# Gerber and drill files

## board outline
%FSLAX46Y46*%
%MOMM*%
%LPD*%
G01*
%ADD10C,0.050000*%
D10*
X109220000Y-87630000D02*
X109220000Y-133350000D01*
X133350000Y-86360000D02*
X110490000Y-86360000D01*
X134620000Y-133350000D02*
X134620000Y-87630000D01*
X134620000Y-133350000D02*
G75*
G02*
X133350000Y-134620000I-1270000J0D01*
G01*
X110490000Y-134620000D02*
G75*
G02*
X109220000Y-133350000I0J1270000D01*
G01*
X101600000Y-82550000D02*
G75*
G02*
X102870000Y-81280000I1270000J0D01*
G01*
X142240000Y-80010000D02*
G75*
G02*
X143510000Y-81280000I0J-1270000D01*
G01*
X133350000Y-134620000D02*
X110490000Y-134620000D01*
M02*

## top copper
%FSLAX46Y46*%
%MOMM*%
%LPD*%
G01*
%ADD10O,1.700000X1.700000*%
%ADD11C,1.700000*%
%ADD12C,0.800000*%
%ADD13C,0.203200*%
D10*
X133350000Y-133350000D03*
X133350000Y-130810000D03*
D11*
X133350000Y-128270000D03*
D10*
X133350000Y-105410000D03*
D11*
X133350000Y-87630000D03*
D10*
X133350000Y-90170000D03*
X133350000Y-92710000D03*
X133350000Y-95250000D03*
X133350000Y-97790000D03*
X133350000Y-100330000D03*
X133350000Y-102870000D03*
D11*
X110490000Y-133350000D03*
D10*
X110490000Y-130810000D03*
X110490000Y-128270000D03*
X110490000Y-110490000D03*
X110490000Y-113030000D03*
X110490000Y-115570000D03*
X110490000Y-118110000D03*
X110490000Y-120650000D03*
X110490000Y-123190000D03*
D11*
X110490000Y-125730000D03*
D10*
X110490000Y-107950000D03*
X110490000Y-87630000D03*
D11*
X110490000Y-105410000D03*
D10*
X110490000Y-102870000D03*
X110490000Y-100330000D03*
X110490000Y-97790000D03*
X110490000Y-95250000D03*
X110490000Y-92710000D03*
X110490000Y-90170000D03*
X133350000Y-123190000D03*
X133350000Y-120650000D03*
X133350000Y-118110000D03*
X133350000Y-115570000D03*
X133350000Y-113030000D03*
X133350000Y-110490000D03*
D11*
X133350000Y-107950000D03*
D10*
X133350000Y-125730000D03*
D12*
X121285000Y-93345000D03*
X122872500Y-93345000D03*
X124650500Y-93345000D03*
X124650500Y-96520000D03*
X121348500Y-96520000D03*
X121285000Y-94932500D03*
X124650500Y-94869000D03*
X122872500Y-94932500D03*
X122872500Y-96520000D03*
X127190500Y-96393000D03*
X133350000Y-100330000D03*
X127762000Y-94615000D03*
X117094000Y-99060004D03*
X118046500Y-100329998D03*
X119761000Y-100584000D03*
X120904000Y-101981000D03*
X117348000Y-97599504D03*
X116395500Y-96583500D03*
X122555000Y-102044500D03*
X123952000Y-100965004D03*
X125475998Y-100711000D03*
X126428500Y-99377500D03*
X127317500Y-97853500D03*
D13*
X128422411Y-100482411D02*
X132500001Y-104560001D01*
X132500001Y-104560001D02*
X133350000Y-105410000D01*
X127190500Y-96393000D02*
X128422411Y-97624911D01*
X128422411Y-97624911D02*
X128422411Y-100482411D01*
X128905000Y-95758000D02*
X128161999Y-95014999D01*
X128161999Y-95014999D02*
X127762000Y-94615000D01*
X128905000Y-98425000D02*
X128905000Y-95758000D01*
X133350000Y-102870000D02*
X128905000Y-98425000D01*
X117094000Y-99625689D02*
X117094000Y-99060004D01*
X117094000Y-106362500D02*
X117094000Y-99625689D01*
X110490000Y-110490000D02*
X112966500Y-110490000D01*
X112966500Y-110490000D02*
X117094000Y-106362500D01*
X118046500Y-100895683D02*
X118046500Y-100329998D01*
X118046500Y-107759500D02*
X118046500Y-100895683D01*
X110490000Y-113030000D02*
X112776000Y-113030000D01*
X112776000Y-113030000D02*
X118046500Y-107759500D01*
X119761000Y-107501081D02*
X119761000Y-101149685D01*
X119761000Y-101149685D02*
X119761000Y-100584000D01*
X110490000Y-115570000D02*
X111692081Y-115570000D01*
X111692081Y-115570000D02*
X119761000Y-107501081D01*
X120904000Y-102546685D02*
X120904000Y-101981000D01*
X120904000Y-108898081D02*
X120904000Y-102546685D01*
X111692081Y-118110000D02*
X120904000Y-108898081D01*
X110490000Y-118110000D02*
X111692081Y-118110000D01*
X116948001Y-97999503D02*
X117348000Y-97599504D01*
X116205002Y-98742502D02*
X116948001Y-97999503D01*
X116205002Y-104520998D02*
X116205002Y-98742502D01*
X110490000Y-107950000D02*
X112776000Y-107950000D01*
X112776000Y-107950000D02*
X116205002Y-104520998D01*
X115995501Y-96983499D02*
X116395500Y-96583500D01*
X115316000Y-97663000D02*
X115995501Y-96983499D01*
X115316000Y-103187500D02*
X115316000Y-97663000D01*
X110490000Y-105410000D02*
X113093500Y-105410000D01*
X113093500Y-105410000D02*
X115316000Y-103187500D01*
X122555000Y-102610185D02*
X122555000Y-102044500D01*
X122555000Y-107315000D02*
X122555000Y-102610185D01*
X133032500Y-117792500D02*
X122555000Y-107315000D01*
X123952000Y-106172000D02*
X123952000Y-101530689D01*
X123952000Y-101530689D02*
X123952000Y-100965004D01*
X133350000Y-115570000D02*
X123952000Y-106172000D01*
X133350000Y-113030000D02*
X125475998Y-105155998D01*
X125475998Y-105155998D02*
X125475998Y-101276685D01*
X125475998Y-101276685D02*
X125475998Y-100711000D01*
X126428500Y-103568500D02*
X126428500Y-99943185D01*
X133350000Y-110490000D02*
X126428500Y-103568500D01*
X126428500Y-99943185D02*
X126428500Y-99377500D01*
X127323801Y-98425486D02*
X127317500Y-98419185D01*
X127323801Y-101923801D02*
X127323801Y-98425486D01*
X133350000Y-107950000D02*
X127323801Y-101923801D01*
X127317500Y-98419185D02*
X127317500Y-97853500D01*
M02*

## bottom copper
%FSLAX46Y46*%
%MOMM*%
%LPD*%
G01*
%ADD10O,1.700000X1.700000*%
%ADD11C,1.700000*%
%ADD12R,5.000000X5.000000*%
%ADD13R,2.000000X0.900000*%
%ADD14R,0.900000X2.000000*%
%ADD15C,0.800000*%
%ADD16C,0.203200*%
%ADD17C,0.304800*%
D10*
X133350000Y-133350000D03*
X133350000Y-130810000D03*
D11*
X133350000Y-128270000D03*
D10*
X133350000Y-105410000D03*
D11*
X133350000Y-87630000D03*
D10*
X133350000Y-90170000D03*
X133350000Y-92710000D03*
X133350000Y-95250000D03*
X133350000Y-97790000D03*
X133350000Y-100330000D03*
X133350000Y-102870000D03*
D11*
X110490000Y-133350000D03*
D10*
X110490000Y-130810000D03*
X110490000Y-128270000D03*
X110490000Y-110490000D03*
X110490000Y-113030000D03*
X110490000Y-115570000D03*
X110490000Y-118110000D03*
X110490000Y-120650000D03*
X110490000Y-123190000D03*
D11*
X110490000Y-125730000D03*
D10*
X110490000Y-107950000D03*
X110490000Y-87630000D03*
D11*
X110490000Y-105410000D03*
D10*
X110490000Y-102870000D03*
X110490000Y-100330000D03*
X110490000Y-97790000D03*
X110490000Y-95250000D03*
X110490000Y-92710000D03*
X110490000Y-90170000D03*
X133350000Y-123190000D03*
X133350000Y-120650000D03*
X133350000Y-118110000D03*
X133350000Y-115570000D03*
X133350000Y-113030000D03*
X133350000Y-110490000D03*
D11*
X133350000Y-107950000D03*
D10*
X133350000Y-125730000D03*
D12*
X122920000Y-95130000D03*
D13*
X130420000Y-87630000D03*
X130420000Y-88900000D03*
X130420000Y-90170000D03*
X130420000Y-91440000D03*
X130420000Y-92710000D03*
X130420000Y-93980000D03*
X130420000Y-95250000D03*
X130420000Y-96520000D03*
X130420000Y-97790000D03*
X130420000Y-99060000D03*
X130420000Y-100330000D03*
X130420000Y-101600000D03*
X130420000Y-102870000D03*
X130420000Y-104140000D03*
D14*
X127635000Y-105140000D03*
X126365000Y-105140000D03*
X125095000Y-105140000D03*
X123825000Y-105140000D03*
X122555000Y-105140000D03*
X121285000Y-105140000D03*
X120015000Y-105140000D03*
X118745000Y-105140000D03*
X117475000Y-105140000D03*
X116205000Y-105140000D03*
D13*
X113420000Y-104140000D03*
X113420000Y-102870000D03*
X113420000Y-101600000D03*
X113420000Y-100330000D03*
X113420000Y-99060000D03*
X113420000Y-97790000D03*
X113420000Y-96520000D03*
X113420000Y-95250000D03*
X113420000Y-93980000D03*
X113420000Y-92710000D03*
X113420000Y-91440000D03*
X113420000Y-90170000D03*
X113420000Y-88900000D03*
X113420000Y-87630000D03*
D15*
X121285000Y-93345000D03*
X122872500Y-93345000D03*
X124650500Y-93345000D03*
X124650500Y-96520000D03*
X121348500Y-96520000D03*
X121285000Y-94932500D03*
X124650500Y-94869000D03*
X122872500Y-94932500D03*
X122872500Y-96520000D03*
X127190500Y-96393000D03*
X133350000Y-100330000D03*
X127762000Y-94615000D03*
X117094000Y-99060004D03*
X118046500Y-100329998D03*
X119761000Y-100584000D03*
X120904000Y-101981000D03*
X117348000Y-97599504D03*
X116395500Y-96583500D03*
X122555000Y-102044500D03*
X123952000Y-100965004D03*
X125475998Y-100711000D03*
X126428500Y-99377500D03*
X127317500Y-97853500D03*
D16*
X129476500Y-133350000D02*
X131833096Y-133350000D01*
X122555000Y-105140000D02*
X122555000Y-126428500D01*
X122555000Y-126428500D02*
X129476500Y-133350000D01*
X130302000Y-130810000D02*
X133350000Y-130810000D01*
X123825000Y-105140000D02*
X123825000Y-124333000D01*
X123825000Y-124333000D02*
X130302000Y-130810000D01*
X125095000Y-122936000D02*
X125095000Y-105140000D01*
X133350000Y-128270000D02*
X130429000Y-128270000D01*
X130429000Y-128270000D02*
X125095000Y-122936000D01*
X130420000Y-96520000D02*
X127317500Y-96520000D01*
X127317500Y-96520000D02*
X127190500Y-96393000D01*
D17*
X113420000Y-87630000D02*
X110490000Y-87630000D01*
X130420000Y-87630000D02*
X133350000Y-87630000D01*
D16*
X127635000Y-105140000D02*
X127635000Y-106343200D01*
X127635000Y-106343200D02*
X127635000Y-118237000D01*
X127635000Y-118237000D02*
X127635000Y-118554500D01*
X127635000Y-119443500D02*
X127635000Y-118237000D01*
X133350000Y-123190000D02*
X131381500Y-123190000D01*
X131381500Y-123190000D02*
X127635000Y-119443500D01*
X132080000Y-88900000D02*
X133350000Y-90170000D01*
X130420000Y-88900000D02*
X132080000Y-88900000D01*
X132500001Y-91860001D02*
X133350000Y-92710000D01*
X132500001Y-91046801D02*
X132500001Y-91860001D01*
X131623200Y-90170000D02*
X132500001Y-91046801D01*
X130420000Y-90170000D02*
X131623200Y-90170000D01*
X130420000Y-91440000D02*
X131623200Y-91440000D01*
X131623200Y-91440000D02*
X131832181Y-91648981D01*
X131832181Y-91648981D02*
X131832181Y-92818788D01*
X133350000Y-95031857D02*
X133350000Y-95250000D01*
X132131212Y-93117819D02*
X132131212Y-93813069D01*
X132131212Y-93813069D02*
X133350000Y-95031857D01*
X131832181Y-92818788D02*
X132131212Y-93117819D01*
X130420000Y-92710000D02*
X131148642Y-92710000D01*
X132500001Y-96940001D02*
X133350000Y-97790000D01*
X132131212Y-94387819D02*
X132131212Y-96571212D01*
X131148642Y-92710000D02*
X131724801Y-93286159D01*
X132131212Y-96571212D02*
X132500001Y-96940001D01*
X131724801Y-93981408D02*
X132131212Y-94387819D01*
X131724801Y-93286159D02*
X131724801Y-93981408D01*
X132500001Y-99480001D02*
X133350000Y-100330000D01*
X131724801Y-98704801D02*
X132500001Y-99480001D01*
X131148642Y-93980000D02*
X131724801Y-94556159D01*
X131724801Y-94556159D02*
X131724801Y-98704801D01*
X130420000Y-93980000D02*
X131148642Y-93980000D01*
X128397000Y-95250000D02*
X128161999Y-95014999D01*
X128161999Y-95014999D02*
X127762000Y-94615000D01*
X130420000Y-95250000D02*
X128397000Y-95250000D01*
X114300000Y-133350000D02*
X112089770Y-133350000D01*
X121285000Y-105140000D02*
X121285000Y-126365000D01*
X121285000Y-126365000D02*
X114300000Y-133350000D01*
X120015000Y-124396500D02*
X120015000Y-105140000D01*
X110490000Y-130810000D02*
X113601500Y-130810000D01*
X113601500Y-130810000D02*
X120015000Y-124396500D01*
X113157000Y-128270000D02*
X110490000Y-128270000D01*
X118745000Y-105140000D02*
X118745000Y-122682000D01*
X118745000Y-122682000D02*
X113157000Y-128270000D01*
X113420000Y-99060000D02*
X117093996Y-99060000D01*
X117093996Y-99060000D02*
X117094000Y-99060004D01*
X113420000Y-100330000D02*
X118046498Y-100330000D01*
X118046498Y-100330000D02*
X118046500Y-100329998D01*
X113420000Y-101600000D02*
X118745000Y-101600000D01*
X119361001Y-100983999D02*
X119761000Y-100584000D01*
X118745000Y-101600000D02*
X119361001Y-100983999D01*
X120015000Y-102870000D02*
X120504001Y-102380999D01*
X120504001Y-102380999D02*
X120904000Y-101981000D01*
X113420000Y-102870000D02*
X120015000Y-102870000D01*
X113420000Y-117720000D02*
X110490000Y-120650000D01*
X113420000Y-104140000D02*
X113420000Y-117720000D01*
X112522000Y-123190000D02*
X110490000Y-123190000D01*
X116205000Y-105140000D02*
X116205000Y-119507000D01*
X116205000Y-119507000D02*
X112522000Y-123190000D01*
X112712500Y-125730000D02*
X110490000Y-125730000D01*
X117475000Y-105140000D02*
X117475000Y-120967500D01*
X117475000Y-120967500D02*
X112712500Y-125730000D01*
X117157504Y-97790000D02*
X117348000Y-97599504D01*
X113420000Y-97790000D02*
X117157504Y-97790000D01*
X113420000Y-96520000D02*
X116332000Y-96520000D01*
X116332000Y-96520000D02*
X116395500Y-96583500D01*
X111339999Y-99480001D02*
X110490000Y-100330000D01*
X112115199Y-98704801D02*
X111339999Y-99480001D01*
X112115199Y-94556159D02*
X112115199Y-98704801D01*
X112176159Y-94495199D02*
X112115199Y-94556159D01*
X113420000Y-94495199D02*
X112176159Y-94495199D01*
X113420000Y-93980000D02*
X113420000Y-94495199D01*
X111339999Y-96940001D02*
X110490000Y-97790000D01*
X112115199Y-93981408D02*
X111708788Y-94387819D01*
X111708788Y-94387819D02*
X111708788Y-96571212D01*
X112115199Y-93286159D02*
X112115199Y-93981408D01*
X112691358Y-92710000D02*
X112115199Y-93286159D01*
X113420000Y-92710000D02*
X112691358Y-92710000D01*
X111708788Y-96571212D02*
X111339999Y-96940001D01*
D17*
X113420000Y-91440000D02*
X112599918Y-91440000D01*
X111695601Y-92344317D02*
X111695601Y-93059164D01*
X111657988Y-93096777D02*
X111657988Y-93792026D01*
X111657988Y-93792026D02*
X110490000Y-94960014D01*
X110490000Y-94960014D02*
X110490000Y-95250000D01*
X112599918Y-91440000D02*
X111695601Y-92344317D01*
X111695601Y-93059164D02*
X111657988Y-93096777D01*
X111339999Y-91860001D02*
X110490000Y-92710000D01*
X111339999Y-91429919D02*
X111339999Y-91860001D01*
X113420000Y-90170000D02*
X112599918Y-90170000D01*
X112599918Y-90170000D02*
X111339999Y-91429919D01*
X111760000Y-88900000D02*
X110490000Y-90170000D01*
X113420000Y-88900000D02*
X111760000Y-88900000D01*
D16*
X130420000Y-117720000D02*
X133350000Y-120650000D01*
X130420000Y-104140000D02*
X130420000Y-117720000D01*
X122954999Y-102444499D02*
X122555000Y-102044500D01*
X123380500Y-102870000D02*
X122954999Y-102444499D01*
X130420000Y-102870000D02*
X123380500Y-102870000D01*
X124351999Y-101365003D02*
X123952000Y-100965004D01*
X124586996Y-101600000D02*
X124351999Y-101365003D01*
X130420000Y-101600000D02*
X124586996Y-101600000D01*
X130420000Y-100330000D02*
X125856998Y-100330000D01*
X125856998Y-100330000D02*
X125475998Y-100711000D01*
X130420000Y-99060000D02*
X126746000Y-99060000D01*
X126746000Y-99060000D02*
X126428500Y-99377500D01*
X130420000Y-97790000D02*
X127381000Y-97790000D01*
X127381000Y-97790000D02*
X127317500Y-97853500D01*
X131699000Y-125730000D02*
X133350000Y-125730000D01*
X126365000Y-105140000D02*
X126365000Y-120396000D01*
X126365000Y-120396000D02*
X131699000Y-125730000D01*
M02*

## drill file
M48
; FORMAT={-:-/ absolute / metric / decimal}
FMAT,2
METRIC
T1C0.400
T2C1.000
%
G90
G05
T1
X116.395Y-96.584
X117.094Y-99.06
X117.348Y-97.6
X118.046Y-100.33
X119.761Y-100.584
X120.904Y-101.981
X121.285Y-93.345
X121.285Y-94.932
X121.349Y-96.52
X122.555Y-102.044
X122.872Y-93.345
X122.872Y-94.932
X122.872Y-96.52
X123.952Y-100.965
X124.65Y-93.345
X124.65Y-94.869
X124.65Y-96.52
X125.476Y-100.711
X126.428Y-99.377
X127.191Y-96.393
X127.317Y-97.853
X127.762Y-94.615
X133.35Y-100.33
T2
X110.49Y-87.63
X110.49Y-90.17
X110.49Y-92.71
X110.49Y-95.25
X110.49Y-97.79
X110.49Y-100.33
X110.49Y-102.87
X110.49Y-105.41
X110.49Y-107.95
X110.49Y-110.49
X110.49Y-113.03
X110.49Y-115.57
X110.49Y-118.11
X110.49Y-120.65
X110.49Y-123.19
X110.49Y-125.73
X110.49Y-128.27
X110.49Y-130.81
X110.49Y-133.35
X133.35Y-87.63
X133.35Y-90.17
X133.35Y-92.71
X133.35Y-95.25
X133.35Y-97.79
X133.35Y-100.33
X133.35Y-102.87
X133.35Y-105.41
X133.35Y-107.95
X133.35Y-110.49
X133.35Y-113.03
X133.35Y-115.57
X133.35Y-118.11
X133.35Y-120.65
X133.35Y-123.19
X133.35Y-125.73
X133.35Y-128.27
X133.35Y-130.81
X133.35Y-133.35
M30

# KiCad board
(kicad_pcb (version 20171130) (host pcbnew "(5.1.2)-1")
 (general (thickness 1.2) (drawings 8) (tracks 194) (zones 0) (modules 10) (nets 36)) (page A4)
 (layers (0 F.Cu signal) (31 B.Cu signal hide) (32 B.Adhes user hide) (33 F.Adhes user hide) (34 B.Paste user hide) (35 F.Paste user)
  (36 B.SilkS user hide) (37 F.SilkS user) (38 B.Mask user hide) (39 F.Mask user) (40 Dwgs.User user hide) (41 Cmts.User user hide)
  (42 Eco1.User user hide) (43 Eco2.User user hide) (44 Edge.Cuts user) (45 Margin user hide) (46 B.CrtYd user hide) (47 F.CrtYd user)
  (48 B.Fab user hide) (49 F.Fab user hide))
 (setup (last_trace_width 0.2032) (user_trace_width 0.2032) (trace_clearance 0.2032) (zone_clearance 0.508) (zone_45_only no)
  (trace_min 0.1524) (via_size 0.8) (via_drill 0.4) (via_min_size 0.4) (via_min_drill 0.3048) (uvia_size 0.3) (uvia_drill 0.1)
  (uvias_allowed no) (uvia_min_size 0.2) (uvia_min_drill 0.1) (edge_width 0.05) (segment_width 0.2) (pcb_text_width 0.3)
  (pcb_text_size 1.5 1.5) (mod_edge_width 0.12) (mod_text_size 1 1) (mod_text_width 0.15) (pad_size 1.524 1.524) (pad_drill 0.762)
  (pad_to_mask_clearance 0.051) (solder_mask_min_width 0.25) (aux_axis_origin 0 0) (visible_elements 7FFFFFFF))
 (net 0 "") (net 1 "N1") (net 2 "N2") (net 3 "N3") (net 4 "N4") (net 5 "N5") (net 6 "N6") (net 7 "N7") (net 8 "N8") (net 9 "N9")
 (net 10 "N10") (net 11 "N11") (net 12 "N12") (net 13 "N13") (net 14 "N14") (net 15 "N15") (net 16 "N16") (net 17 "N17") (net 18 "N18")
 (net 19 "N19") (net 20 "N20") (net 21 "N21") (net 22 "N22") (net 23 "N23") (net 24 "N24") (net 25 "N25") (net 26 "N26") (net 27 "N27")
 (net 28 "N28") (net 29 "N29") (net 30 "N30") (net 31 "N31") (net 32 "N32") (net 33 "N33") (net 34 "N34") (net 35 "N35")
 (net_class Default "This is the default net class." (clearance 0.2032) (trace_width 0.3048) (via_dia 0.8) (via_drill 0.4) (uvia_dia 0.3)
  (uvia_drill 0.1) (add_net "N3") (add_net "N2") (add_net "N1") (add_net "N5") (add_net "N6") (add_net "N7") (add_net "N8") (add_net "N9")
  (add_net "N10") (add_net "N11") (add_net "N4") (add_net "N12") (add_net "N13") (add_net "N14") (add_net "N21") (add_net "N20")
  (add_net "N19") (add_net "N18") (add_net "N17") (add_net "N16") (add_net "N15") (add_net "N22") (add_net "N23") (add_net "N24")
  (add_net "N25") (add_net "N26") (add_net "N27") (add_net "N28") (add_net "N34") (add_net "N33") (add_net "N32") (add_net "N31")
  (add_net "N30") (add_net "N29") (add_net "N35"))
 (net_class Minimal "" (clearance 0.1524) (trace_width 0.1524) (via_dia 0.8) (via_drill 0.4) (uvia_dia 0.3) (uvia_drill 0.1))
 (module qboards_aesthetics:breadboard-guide (layer F.Cu) (at 97.79 90.17)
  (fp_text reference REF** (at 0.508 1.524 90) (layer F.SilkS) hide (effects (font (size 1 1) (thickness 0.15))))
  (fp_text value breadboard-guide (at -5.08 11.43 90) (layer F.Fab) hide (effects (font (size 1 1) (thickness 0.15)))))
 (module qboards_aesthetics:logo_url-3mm (layer F.Cu) (at 117.602 117.983)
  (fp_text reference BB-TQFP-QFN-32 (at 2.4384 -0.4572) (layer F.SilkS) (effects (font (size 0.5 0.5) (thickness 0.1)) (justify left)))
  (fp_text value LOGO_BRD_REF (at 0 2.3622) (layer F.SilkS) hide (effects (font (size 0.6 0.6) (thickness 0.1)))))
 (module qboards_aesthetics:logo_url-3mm (layer B.Cu) (at 126.492 117.983 180)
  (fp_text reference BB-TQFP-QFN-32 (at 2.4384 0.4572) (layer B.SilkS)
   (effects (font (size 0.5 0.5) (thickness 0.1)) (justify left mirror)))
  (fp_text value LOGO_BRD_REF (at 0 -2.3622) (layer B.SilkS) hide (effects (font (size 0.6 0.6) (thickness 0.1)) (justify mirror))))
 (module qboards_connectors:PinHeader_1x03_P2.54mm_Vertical (layer F.Cu) (at 133.35 128.27)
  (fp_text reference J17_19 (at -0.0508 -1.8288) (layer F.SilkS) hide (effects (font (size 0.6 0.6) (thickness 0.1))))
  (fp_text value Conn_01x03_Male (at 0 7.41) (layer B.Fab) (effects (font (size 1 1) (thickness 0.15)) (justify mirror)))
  (pad 3 thru_hole oval (at 0 5.08) (size 1.7 1.7) (drill 1) (layers *.Cu *.Mask) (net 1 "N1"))
  (pad 2 thru_hole oval (at 0 2.54) (size 1.7 1.7) (drill 1) (layers *.Cu *.Mask) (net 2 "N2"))
  (pad 1 thru_hole circle (at 0 0) (size 1.7 1.7) (drill 1) (layers *.Cu *.Mask) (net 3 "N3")))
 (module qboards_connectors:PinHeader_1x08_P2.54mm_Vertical (layer F.Cu) (at 133.35 87.63)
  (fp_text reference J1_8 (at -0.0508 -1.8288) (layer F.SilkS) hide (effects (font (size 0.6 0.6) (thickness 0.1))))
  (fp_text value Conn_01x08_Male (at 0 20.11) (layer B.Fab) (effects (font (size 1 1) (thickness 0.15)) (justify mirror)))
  (pad 8 thru_hole oval (at 0 17.78) (size 1.7 1.7) (drill 1) (layers *.Cu *.Mask) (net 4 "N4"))
  (pad 1 thru_hole circle (at 0 0) (size 1.7 1.7) (drill 1) (layers *.Cu *.Mask) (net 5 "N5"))
  (pad 2 thru_hole oval (at 0 2.54) (size 1.7 1.7) (drill 1) (layers *.Cu *.Mask) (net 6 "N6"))
  (pad 3 thru_hole oval (at 0 5.08) (size 1.7 1.7) (drill 1) (layers *.Cu *.Mask) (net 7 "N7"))
  (pad 4 thru_hole oval (at 0 7.62) (size 1.7 1.7) (drill 1) (layers *.Cu *.Mask) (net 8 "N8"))
  (pad 5 thru_hole oval (at 0 10.16) (size 1.7 1.7) (drill 1) (layers *.Cu *.Mask) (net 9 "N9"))
  (pad 6 thru_hole oval (at 0 12.7) (size 1.7 1.7) (drill 1) (layers *.Cu *.Mask) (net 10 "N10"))
  (pad 7 thru_hole oval (at 0 15.24) (size 1.7 1.7) (drill 1) (layers *.Cu *.Mask) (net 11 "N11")))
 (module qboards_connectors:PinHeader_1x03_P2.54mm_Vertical (layer F.Cu) (at 110.49 133.35 180)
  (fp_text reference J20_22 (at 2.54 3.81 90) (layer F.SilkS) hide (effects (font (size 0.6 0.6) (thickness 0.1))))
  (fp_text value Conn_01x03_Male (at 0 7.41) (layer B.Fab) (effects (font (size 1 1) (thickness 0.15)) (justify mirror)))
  (pad 1 thru_hole circle (at 0 0 180) (size 1.7 1.7) (drill 1) (layers *.Cu *.Mask) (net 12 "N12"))
  (pad 2 thru_hole oval (at 0 2.54 180) (size 1.7 1.7) (drill 1) (layers *.Cu *.Mask) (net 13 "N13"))
  (pad 3 thru_hole oval (at 0 5.08 180) (size 1.7 1.7) (drill 1) (layers *.Cu *.Mask) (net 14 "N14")))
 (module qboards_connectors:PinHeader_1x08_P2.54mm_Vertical (layer F.Cu) (at 110.49 125.73 180)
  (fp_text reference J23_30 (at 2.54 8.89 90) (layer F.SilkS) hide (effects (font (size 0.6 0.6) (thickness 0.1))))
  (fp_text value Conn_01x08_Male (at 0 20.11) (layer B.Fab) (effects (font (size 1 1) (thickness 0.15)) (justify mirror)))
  (pad 7 thru_hole oval (at 0 15.24 180) (size 1.7 1.7) (drill 1) (layers *.Cu *.Mask) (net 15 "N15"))
  (pad 6 thru_hole oval (at 0 12.7 180) (size 1.7 1.7) (drill 1) (layers *.Cu *.Mask) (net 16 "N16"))
  (pad 5 thru_hole oval (at 0 10.16 180) (size 1.7 1.7) (drill 1) (layers *.Cu *.Mask) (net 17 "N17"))
  (pad 4 thru_hole oval (at 0 7.62 180) (size 1.7 1.7) (drill 1) (layers *.Cu *.Mask) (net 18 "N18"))
  (pad 3 thru_hole oval (at 0 5.08 180) (size 1.7 1.7) (drill 1) (layers *.Cu *.Mask) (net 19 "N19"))
  (pad 2 thru_hole oval (at 0 2.54 180) (size 1.7 1.7) (drill 1) (layers *.Cu *.Mask) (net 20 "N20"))
  (pad 1 thru_hole circle (at 0 0 180) (size 1.7 1.7) (drill 1) (layers *.Cu *.Mask) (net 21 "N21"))
  (pad 8 thru_hole oval (at 0 17.78 180) (size 1.7 1.7) (drill 1) (layers *.Cu *.Mask) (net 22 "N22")))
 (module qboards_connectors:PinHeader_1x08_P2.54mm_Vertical (layer F.Cu) (at 110.49 105.41 180)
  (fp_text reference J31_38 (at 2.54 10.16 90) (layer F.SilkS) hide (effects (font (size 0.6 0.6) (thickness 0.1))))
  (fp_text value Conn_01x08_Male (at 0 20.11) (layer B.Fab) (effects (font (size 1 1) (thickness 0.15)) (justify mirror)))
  (pad 8 thru_hole oval (at 0 17.78 180) (size 1.7 1.7) (drill 1) (layers *.Cu *.Mask) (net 5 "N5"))
  (pad 1 thru_hole circle (at 0 0 180) (size 1.7 1.7) (drill 1) (layers *.Cu *.Mask) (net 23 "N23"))
  (pad 2 thru_hole oval (at 0 2.54 180) (size 1.7 1.7) (drill 1) (layers *.Cu *.Mask))
  (pad 3 thru_hole oval (at 0 5.08 180) (size 1.7 1.7) (drill 1) (layers *.Cu *.Mask) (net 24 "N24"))
  (pad 4 thru_hole oval (at 0 7.62 180) (size 1.7 1.7) (drill 1) (layers *.Cu *.Mask) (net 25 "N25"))
  (pad 5 thru_hole oval (at 0 10.16 180) (size 1.7 1.7) (drill 1) (layers *.Cu *.Mask) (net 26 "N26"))
  (pad 6 thru_hole oval (at 0 12.7 180) (size 1.7 1.7) (drill 1) (layers *.Cu *.Mask) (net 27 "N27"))
  (pad 7 thru_hole oval (at 0 15.24 180) (size 1.7 1.7) (drill 1) (layers *.Cu *.Mask) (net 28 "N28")))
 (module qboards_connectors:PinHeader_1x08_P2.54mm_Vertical (layer F.Cu) (at 133.35 107.95)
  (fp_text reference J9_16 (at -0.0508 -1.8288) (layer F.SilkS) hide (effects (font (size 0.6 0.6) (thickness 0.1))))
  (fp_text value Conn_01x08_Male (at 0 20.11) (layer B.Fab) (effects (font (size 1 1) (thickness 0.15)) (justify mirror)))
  (pad 7 thru_hole oval (at 0 15.24) (size 1.7 1.7) (drill 1) (layers *.Cu *.Mask) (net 5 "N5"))
  (pad 6 thru_hole oval (at 0 12.7) (size 1.7 1.7) (drill 1) (layers *.Cu *.Mask) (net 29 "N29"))
  (pad 5 thru_hole oval (at 0 10.16) (size 1.7 1.7) (drill 1) (layers *.Cu *.Mask) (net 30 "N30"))
  (pad 4 thru_hole oval (at 0 7.62) (size 1.7 1.7) (drill 1) (layers *.Cu *.Mask) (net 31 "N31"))
  (pad 3 thru_hole oval (at 0 5.08) (size 1.7 1.7) (drill 1) (layers *.Cu *.Mask) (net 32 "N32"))
  (pad 2 thru_hole oval (at 0 2.54) (size 1.7 1.7) (drill 1) (layers *.Cu *.Mask) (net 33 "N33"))
  (pad 1 thru_hole circle (at 0 0) (size 1.7 1.7) (drill 1) (layers *.Cu *.Mask) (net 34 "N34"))
  (pad 8 thru_hole oval (at 0 17.78) (size 1.7 1.7) (drill 1) (layers *.Cu *.Mask) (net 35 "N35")))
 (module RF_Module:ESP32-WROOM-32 (layer B.Cu) (at 121.92 95.885 180)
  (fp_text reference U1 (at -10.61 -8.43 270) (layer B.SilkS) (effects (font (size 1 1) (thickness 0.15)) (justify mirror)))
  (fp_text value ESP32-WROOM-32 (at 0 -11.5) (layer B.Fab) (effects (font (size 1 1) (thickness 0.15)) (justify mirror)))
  (pad 39 smd rect (at -1 0.755 180) (size 5 5) (layers B.Cu B.Paste B.Mask))
  (pad 1 smd rect (at -8.5 8.255 180) (size 2 0.9) (layers B.Cu B.Paste B.Mask) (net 5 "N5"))
  (pad 2 smd rect (at -8.5 6.985 180) (size 2 0.9) (layers B.Cu B.Paste B.Mask) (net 6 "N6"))
  (pad 3 smd rect (at -8.5 5.715 180) (size 2 0.9) (layers B.Cu B.Paste B.Mask) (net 7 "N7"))
  (pad 4 smd rect (at -8.5 4.445 180) (size 2 0.9) (layers B.Cu B.Paste B.Mask) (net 8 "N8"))
  (pad 5 smd rect (at -8.5 3.175 180) (size 2 0.9) (layers B.Cu B.Paste B.Mask) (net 9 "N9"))
  (pad 6 smd rect (at -8.5 1.905 180) (size 2 0.9) (layers B.Cu B.Paste B.Mask) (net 10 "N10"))
  (pad 7 smd rect (at -8.5 0.635 180) (size 2 0.9) (layers B.Cu B.Paste B.Mask) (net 11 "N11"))
  (pad 8 smd rect (at -8.5 -0.635 180) (size 2 0.9) (layers B.Cu B.Paste B.Mask) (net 4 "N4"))
  (pad 9 smd rect (at -8.5 -1.905 180) (size 2 0.9) (layers B.Cu B.Paste B.Mask) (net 34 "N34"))
  (pad 10 smd rect (at -8.5 -3.175 180) (size 2 0.9) (layers B.Cu B.Paste B.Mask) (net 33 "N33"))
  (pad 11 smd rect (at -8.5 -4.445 180) (size 2 0.9) (layers B.Cu B.Paste B.Mask) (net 32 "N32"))
  (pad 12 smd rect (at -8.5 -5.715 180) (size 2 0.9) (layers B.Cu B.Paste B.Mask) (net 31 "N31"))
  (pad 13 smd rect (at -8.5 -6.985 180) (size 2 0.9) (layers B.Cu B.Paste B.Mask) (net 30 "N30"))
  (pad 14 smd rect (at -8.5 -8.255 180) (size 2 0.9) (layers B.Cu B.Paste B.Mask) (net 29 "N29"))
  (pad 15 smd rect (at -5.715 -9.255 90) (size 2 0.9) (layers B.Cu B.Paste B.Mask) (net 5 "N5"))
  (pad 16 smd rect (at -4.445 -9.255 90) (size 2 0.9) (layers B.Cu B.Paste B.Mask) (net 35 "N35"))
  (pad 17 smd rect (at -3.175 -9.255 90) (size 2 0.9) (layers B.Cu B.Paste B.Mask) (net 3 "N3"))
  (pad 18 smd rect (at -1.905 -9.255 90) (size 2 0.9) (layers B.Cu B.Paste B.Mask) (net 2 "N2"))
  (pad 19 smd rect (at -0.635 -9.255 90) (size 2 0.9) (layers B.Cu B.Paste B.Mask) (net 1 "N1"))
  (pad 20 smd rect (at 0.635 -9.255 90) (size 2 0.9) (layers B.Cu B.Paste B.Mask) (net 12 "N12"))
  (pad 21 smd rect (at 1.905 -9.255 90) (size 2 0.9) (layers B.Cu B.Paste B.Mask) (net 13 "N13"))
  (pad 22 smd rect (at 3.175 -9.255 90) (size 2 0.9) (layers B.Cu B.Paste B.Mask) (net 14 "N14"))
  (pad 23 smd rect (at 4.445 -9.255 90) (size 2 0.9) (layers B.Cu B.Paste B.Mask) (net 21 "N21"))
  (pad 24 smd rect (at 5.715 -9.255 90) (size 2 0.9) (layers B.Cu B.Paste B.Mask) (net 20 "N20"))
  (pad 25 smd rect (at 8.5 -8.255 180) (size 2 0.9) (layers B.Cu B.Paste B.Mask) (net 19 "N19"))
  (pad 26 smd rect (at 8.5 -6.985 180) (size 2 0.9) (layers B.Cu B.Paste B.Mask) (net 18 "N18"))
  (pad 27 smd rect (at 8.5 -5.715 180) (size 2 0.9) (layers B.Cu B.Paste B.Mask) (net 17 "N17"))
  (pad 28 smd rect (at 8.5 -4.445 180) (size 2 0.9) (layers B.Cu B.Paste B.Mask) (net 16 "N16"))
  (pad 29 smd rect (at 8.5 -3.175 180) (size 2 0.9) (layers B.Cu B.Paste B.Mask) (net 15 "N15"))
  (pad 30 smd rect (at 8.5 -1.905 180) (size 2 0.9) (layers B.Cu B.Paste B.Mask) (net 22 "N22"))
  (pad 31 smd rect (at 8.5 -0.635 180) (size 2 0.9) (layers B.Cu B.Paste B.Mask) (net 23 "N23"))
  (pad 32 smd rect (at 8.5 0.635 180) (size 2 0.9) (layers B.Cu B.Paste B.Mask))
  (pad 33 smd rect (at 8.5 1.905 180) (size 2 0.9) (layers B.Cu B.Paste B.Mask) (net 24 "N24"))
  (pad 34 smd rect (at 8.5 3.175 180) (size 2 0.9) (layers B.Cu B.Paste B.Mask) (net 25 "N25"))
  (pad 35 smd rect (at 8.5 4.445 180) (size 2 0.9) (layers B.Cu B.Paste B.Mask) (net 26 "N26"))
  (pad 36 smd rect (at 8.5 5.715 180) (size 2 0.9) (layers B.Cu B.Paste B.Mask) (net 27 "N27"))
  (pad 37 smd rect (at 8.5 6.985 180) (size 2 0.9) (layers B.Cu B.Paste B.Mask) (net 28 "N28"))
  (pad 38 smd rect (at 8.5 8.255 180) (size 2 0.9) (layers B.Cu B.Paste B.Mask) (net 5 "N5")))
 (gr_line (start 109.22 87.63) (end 109.22 133.35) (layer Edge.Cuts) (width 0.05))
 (gr_line (start 133.35 86.36) (end 110.49 86.36) (layer Edge.Cuts) (width 0.05))
 (gr_line (start 134.62 133.35) (end 134.62 87.63) (layer Edge.Cuts) (width 0.05))
 (gr_arc (start 133.35 133.35) (end 133.35 134.62) (angle -90) (layer Edge.Cuts) (width 0.05))
 (gr_arc (start 110.49 133.35) (end 109.22 133.35) (angle -90) (layer Edge.Cuts) (width 0.05))
 (gr_arc (start 102.87 82.55) (end 102.87 81.28) (angle -90) (layer Edge.Cuts) (width 0.05))
 (gr_arc (start 142.24 81.28) (end 143.51 81.28) (angle -90) (layer Edge.Cuts) (width 0.05))
 (gr_line (start 133.35 134.62) (end 110.49 134.62) (layer Edge.Cuts) (width 0.05))
 (via (at 121.285 93.345) (size 0.8) (drill 0.4) (layers F.Cu B.Cu) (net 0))
 (via (at 122.8725 93.345) (size 0.8) (drill 0.4) (layers F.Cu B.Cu) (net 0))
 (via (at 124.6505 93.345) (size 0.8) (drill 0.4) (layers F.Cu B.Cu) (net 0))
 (via (at 124.6505 96.52) (size 0.8) (drill 0.4) (layers F.Cu B.Cu) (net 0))
 (via (at 121.3485 96.52) (size 0.8) (drill 0.4) (layers F.Cu B.Cu) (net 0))
 (via (at 121.285 94.9325) (size 0.8) (drill 0.4) (layers F.Cu B.Cu) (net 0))
 (via (at 124.6505 94.869) (size 0.8) (drill 0.4) (layers F.Cu B.Cu) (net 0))
 (via (at 122.8725 94.9325) (size 0.8) (drill 0.4) (layers F.Cu B.Cu) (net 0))
 (via (at 122.8725 96.52) (size 0.8) (drill 0.4) (layers F.Cu B.Cu) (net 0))
 (segment (start 129.4765 133.35) (end 131.833096 133.35) (width 0.2032) (layer B.Cu) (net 1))
 (segment (start 122.555 105.14) (end 122.555 126.4285) (width 0.2032) (layer B.Cu) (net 1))
 (segment (start 122.555 126.4285) (end 129.4765 133.35) (width 0.2032) (layer B.Cu) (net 1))
 (segment (start 130.302 130.81) (end 133.35 130.81) (width 0.2032) (layer B.Cu) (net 2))
 (segment (start 123.825 105.14) (end 123.825 124.333) (width 0.2032) (layer B.Cu) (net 2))
 (segment (start 123.825 124.333) (end 130.302 130.81) (width 0.2032) (layer B.Cu) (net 2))
 (segment (start 125.095 122.936) (end 125.095 105.14) (width 0.2032) (layer B.Cu) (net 3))
 (segment (start 133.35 128.27) (end 130.429 128.27) (width 0.2032) (layer B.Cu) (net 3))
 (segment (start 130.429 128.27) (end 125.095 122.936) (width 0.2032) (layer B.Cu) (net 3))
 (via (at 127.1905 96.393) (size 0.8) (drill 0.4) (layers F.Cu B.Cu) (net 4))
 (segment (start 130.42 96.52) (end 127.3175 96.52) (width 0.2032) (layer B.Cu) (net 4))
 (segment (start 127.3175 96.52) (end 127.1905 96.393) (width 0.2032) (layer B.Cu) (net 4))
 (segment (start 128.422411 100.482411) (end 132.500001 104.560001) (width 0.2032) (layer F.Cu) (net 4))
 (segment (start 132.500001 104.560001) (end 133.35 105.41) (width 0.2032) (layer F.Cu) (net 4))
 (segment (start 127.1905 96.393) (end 128.422411 97.624911) (width 0.2032) (layer F.Cu) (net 4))
 (segment (start 128.422411 97.624911) (end 128.422411 100.482411) (width 0.2032) (layer F.Cu) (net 4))
 (segment (start 113.42 87.63) (end 110.49 87.63) (width 0.3048) (layer B.Cu) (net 5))
 (segment (start 130.42 87.63) (end 133.35 87.63) (width 0.3048) (layer B.Cu) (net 5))
 (segment (start 127.635 105.14) (end 127.635 106.3432) (width 0.2032) (layer B.Cu) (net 5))
 (segment (start 127.635 106.3432) (end 127.635 118.237) (width 0.2032) (layer B.Cu) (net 5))
 (segment (start 127.635 118.237) (end 127.635 118.5545) (width 0.2032) (layer B.Cu) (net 5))
 (segment (start 127.635 119.4435) (end 127.635 118.237) (width 0.2032) (layer B.Cu) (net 5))
 (segment (start 133.35 123.19) (end 131.3815 123.19) (width 0.2032) (layer B.Cu) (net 5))
 (segment (start 131.3815 123.19) (end 127.635 119.4435) (width 0.2032) (layer B.Cu) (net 5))
 (segment (start 132.08 88.9) (end 133.35 90.17) (width 0.2032) (layer B.Cu) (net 6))
 (segment (start 130.42 88.9) (end 132.08 88.9) (width 0.2032) (layer B.Cu) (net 6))
 (segment (start 132.500001 91.860001) (end 133.35 92.71) (width 0.2032) (layer B.Cu) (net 7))
 (segment (start 132.500001 91.046801) (end 132.500001 91.860001) (width 0.2032) (layer B.Cu) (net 7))
 (segment (start 131.6232 90.17) (end 132.500001 91.046801) (width 0.2032) (layer B.Cu) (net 7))
 (segment (start 130.42 90.17) (end 131.6232 90.17) (width 0.2032) (layer B.Cu) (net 7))
 (segment (start 130.42 91.44) (end 131.6232 91.44) (width 0.2032) (layer B.Cu) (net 8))
 (segment (start 131.6232 91.44) (end 131.832181 91.648981) (width 0.2032) (layer B.Cu) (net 8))
 (segment (start 131.832181 91.648981) (end 131.832181 92.818788) (width 0.2032) (layer B.Cu) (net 8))
 (segment (start 133.35 95.031857) (end 133.35 95.25) (width 0.2032) (layer B.Cu) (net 8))
 (segment (start 132.131212 93.117819) (end 132.131212 93.813069) (width 0.2032) (layer B.Cu) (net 8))
 (segment (start 132.131212 93.813069) (end 133.35 95.031857) (width 0.2032) (layer B.Cu) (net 8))
 (segment (start 131.832181 92.818788) (end 132.131212 93.117819) (width 0.2032) (layer B.Cu) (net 8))
 (segment (start 130.42 92.71) (end 131.148642 92.71) (width 0.2032) (layer B.Cu) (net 9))
 (segment (start 132.500001 96.940001) (end 133.35 97.79) (width 0.2032) (layer B.Cu) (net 9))
 (segment (start 132.131212 94.387819) (end 132.131212 96.571212) (width 0.2032) (layer B.Cu) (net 9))
 (segment (start 131.148642 92.71) (end 131.724801 93.286159) (width 0.2032) (layer B.Cu) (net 9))
 (segment (start 132.131212 96.571212) (end 132.500001 96.940001) (width 0.2032) (layer B.Cu) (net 9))
 (segment (start 131.724801 93.981408) (end 132.131212 94.387819) (width 0.2032) (layer B.Cu) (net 9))
 (segment (start 131.724801 93.286159) (end 131.724801 93.981408) (width 0.2032) (layer B.Cu) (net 9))
 (via (at 133.35 100.33) (size 0.8) (drill 0.4) (layers F.Cu B.Cu) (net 10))
 (segment (start 132.500001 99.480001) (end 133.35 100.33) (width 0.2032) (layer B.Cu) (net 10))
 (segment (start 131.724801 98.704801) (end 132.500001 99.480001) (width 0.2032) (layer B.Cu) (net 10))
 (segment (start 131.148642 93.98) (end 131.724801 94.556159) (width 0.2032) (layer B.Cu) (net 10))
 (segment (start 131.724801 94.556159) (end 131.724801 98.704801) (width 0.2032) (layer B.Cu) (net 10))
 (segment (start 130.42 93.98) (end 131.148642 93.98) (width 0.2032) (layer B.Cu) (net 10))
 (segment (start 128.397 95.25) (end 128.161999 95.014999) (width 0.2032) (layer B.Cu) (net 11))
 (segment (start 128.161999 95.014999) (end 127.762 94.615) (width 0.2032) (layer B.Cu) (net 11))
 (segment (start 130.42 95.25) (end 128.397 95.25) (width 0.2032) (layer B.Cu) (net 11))
 (via (at 127.762 94.615) (size 0.8) (drill 0.4) (layers F.Cu B.Cu) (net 11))
 (segment (start 128.905 95.758) (end 128.161999 95.014999) (width 0.2032) (layer F.Cu) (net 11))
 (segment (start 128.161999 95.014999) (end 127.762 94.615) (width 0.2032) (layer F.Cu) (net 11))
 (segment (start 128.905 98.425) (end 128.905 95.758) (width 0.2032) (layer F.Cu) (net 11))
 (segment (start 133.35 102.87) (end 128.905 98.425) (width 0.2032) (layer F.Cu) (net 11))
 (segment (start 114.3 133.35) (end 112.08977 133.35) (width 0.2032) (layer B.Cu) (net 12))
 (segment (start 121.285 105.14) (end 121.285 126.365) (width 0.2032) (layer B.Cu) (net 12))
 (segment (start 121.285 126.365) (end 114.3 133.35) (width 0.2032) (layer B.Cu) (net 12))
 (segment (start 120.015 124.3965) (end 120.015 105.14) (width 0.2032) (layer B.Cu) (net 13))
 (segment (start 110.49 130.81) (end 113.6015 130.81) (width 0.2032) (layer B.Cu) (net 13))
 (segment (start 113.6015 130.81) (end 120.015 124.3965) (width 0.2032) (layer B.Cu) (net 13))
 (segment (start 113.157 128.27) (end 110.49 128.27) (width 0.2032) (layer B.Cu) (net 14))
 (segment (start 118.745 105.14) (end 118.745 122.682) (width 0.2032) (layer B.Cu) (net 14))
 (segment (start 118.745 122.682) (end 113.157 128.27) (width 0.2032) (layer B.Cu) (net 14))
 (via (at 117.094 99.060004) (size 0.8) (drill 0.4) (layers F.Cu B.Cu) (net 15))
 (segment (start 113.42 99.06) (end 117.093996 99.06) (width 0.2032) (layer B.Cu) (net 15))
 (segment (start 117.093996 99.06) (end 117.094 99.060004) (width 0.2032) (layer B.Cu) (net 15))
 (segment (start 117.094 99.625689) (end 117.094 99.060004) (width 0.2032) (layer F.Cu) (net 15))
 (segment (start 117.094 106.3625) (end 117.094 99.625689) (width 0.2032) (layer F.Cu) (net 15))
 (segment (start 110.49 110.49) (end 112.9665 110.49) (width 0.2032) (layer F.Cu) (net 15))
 (segment (start 112.9665 110.49) (end 117.094 106.3625) (width 0.2032) (layer F.Cu) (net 15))
 (via (at 118.0465 100.329998) (size 0.8) (drill 0.4) (layers F.Cu B.Cu) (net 16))
 (segment (start 113.42 100.33) (end 118.046498 100.33) (width 0.2032) (layer B.Cu) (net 16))
 (segment (start 118.046498 100.33) (end 118.0465 100.329998) (width 0.2032) (layer B.Cu) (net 16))
 (segment (start 118.0465 100.895683) (end 118.0465 100.329998) (width 0.2032) (layer F.Cu) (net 16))
 (segment (start 118.0465 107.7595) (end 118.0465 100.895683) (width 0.2032) (layer F.Cu) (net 16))
 (segment (start 110.49 113.03) (end 112.776 113.03) (width 0.2032) (layer F.Cu) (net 16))
 (segment (start 112.776 113.03) (end 118.0465 107.7595) (width 0.2032) (layer F.Cu) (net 16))
 (via (at 119.761 100.584) (size 0.8) (drill 0.4) (layers F.Cu B.Cu) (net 17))
 (segment (start 113.42 101.6) (end 118.745 101.6) (width 0.2032) (layer B.Cu) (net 17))
 (segment (start 119.761 107.501081) (end 119.761 101.149685) (width 0.2032) (layer F.Cu) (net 17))
 (segment (start 119.761 101.149685) (end 119.761 100.584) (width 0.2032) (layer F.Cu) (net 17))
 (segment (start 110.49 115.57) (end 111.692081 115.57) (width 0.2032) (layer F.Cu) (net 17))
 (segment (start 111.692081 115.57) (end 119.761 107.501081) (width 0.2032) (layer F.Cu) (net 17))
 (segment (start 119.361001 100.983999) (end 119.761 100.584) (width 0.2032) (layer B.Cu) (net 17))
 (segment (start 118.745 101.6) (end 119.361001 100.983999) (width 0.2032) (layer B.Cu) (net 17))
 (via (at 120.904 101.981) (size 0.8) (drill 0.4) (layers F.Cu B.Cu) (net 18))
 (segment (start 120.015 102.87) (end 120.504001 102.380999) (width 0.2032) (layer B.Cu) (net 18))
 (segment (start 120.904 102.546685) (end 120.904 101.981) (width 0.2032) (layer F.Cu) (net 18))
 (segment (start 120.904 108.898081) (end 120.904 102.546685) (width 0.2032) (layer F.Cu) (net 18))
 (segment (start 111.692081 118.11) (end 120.904 108.898081) (width 0.2032) (layer F.Cu) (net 18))
 (segment (start 110.49 118.11) (end 111.692081 118.11) (width 0.2032) (layer F.Cu) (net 18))
 (segment (start 120.504001 102.380999) (end 120.904 101.981) (width 0.2032) (layer B.Cu) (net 18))
 (segment (start 113.42 102.87) (end 120.015 102.87) (width 0.2032) (layer B.Cu) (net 18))
 (segment (start 113.42 117.72) (end 110.49 120.65) (width 0.2032) (layer B.Cu) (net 19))
 (segment (start 113.42 104.14) (end 113.42 117.72) (width 0.2032) (layer B.Cu) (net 19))
 (segment (start 112.522 123.19) (end 110.49 123.19) (width 0.2032) (layer B.Cu) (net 20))
 (segment (start 116.205 105.14) (end 116.205 119.507) (width 0.2032) (layer B.Cu) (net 20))
 (segment (start 116.205 119.507) (end 112.522 123.19) (width 0.2032) (layer B.Cu) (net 20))
 (segment (start 112.7125 125.73) (end 110.49 125.73) (width 0.2032) (layer B.Cu) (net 21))
 (segment (start 117.475 105.14) (end 117.475 120.9675) (width 0.2032) (layer B.Cu) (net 21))
 (segment (start 117.475 120.9675) (end 112.7125 125.73) (width 0.2032) (layer B.Cu) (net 21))
 (via (at 117.348 97.599504) (size 0.8) (drill 0.4) (layers F.Cu B.Cu) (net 22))
 (segment (start 117.157504 97.79) (end 117.348 97.599504) (width 0.2032) (layer B.Cu) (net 22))
 (segment (start 113.42 97.79) (end 117.157504 97.79) (width 0.2032) (layer B.Cu) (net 22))
 (segment (start 116.948001 97.999503) (end 117.348 97.599504) (width 0.2032) (layer F.Cu) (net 22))
 (segment (start 116.205002 98.742502) (end 116.948001 97.999503) (width 0.2032) (layer F.Cu) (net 22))
 (segment (start 116.205002 104.520998) (end 116.205002 98.742502) (width 0.2032) (layer F.Cu) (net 22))
 (segment (start 110.49 107.95) (end 112.776 107.95) (width 0.2032) (layer F.Cu) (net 22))
 (segment (start 112.776 107.95) (end 116.205002 104.520998) (width 0.2032) (layer F.Cu) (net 22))
 (segment (start 113.42 96.52) (end 116.332 96.52) (width 0.2032) (layer B.Cu) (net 23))
 (segment (start 116.332 96.52) (end 116.3955 96.5835) (width 0.2032) (layer B.Cu) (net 23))
 (via (at 116.3955 96.5835) (size 0.8) (drill 0.4) (layers F.Cu B.Cu) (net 23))
 (segment (start 115.995501 96.983499) (end 116.3955 96.5835) (width 0.2032) (layer F.Cu) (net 23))
 (segment (start 115.316 97.663) (end 115.995501 96.983499) (width 0.2032) (layer F.Cu) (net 23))
 (segment (start 115.316 103.1875) (end 115.316 97.663) (width 0.2032) (layer F.Cu) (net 23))
 (segment (start 110.49 105.41) (end 113.0935 105.41) (width 0.2032) (layer F.Cu) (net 23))
 (segment (start 113.0935 105.41) (end 115.316 103.1875) (width 0.2032) (layer F.Cu) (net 23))
 (segment (start 111.339999 99.480001) (end 110.49 100.33) (width 0.2032) (layer B.Cu) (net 24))
 (segment (start 112.115199 98.704801) (end 111.339999 99.480001) (width 0.2032) (layer B.Cu) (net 24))
 (segment (start 112.115199 94.556159) (end 112.115199 98.704801) (width 0.2032) (layer B.Cu) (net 24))
 (segment (start 112.176159 94.495199) (end 112.115199 94.556159) (width 0.2032) (layer B.Cu) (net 24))
 (segment (start 113.42 94.495199) (end 112.176159 94.495199) (width 0.2032) (layer B.Cu) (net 24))
 (segment (start 113.42 93.98) (end 113.42 94.495199) (width 0.2032) (layer B.Cu) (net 24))
 (segment (start 111.339999 96.940001) (end 110.49 97.79) (width 0.2032) (layer B.Cu) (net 25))
 (segment (start 112.115199 93.981408) (end 111.708788 94.387819) (width 0.2032) (layer B.Cu) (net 25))
 (segment (start 111.708788 94.387819) (end 111.708788 96.571212) (width 0.2032) (layer B.Cu) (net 25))
 (segment (start 112.115199 93.286159) (end 112.115199 93.981408) (width 0.2032) (layer B.Cu) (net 25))
 (segment (start 112.691358 92.71) (end 112.115199 93.286159) (width 0.2032) (layer B.Cu) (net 25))
 (segment (start 113.42 92.71) (end 112.691358 92.71) (width 0.2032) (layer B.Cu) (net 25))
 (segment (start 111.708788 96.571212) (end 111.339999 96.940001) (width 0.2032) (layer B.Cu) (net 25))
 (segment (start 113.42 91.44) (end 112.599918 91.44) (width 0.3048) (layer B.Cu) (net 26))
 (segment (start 111.695601 92.344317) (end 111.695601 93.059164) (width 0.3048) (layer B.Cu) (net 26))
 (segment (start 111.657988 93.096777) (end 111.657988 93.792026) (width 0.3048) (layer B.Cu) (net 26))
 (segment (start 111.657988 93.792026) (end 110.49 94.960014) (width 0.3048) (layer B.Cu) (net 26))
 (segment (start 110.49 94.960014) (end 110.49 95.25) (width 0.3048) (layer B.Cu) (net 26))
 (segment (start 112.599918 91.44) (end 111.695601 92.344317) (width 0.3048) (layer B.Cu) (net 26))
 (segment (start 111.695601 93.059164) (end 111.657988 93.096777) (width 0.3048) (layer B.Cu) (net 26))
 (segment (start 111.339999 91.860001) (end 110.49 92.71) (width 0.3048) (layer B.Cu) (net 27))
 (segment (start 111.339999 91.429919) (end 111.339999 91.860001) (width 0.3048) (layer B.Cu) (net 27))
 (segment (start 113.42 90.17) (end 112.599918 90.17) (width 0.3048) (layer B.Cu) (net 27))
 (segment (start 112.599918 90.17) (end 111.339999 91.429919) (width 0.3048) (layer B.Cu) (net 27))
 (segment (start 111.76 88.9) (end 110.49 90.17) (width 0.3048) (layer B.Cu) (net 28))
 (segment (start 113.42 88.9) (end 111.76 88.9) (width 0.3048) (layer B.Cu) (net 28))
 (segment (start 130.42 117.72) (end 133.35 120.65) (width 0.2032) (layer B.Cu) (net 29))
 (segment (start 130.42 104.14) (end 130.42 117.72) (width 0.2032) (layer B.Cu) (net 29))
 (segment (start 122.954999 102.444499) (end 122.555 102.0445) (width 0.2032) (layer B.Cu) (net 30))
 (segment (start 123.3805 102.87) (end 122.954999 102.444499) (width 0.2032) (layer B.Cu) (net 30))
 (segment (start 122.555 102.610185) (end 122.555 102.0445) (width 0.2032) (layer F.Cu) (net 30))
 (segment (start 122.555 107.315) (end 122.555 102.610185) (width 0.2032) (layer F.Cu) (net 30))
 (via (at 122.555 102.0445) (size 0.8) (drill 0.4) (layers F.Cu B.Cu) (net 30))
 (segment (start 130.42 102.87) (end 123.3805 102.87) (width 0.2032) (layer B.Cu) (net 30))
 (segment (start 133.0325 117.7925) (end 122.555 107.315) (width 0.2032) (layer F.Cu) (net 30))
 (via (at 123.952 100.965004) (size 0.8) (drill 0.4) (layers F.Cu B.Cu) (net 31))
 (segment (start 123.952 106.172) (end 123.952 101.530689) (width 0.2032) (layer F.Cu) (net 31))
 (segment (start 123.952 101.530689) (end 123.952 100.965004) (width 0.2032) (layer F.Cu) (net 31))
 (segment (start 133.35 115.57) (end 123.952 106.172) (width 0.2032) (layer F.Cu) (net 31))
 (segment (start 124.351999 101.365003) (end 123.952 100.965004) (width 0.2032) (layer B.Cu) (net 31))
 (segment (start 124.586996 101.6) (end 124.351999 101.365003) (width 0.2032) (layer B.Cu) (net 31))
 (segment (start 130.42 101.6) (end 124.586996 101.6) (width 0.2032) (layer B.Cu) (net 31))
 (via (at 125.475998 100.711) (size 0.8) (drill 0.4) (layers F.Cu B.Cu) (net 32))
 (segment (start 130.42 100.33) (end 125.856998 100.33) (width 0.2032) (layer B.Cu) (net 32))
 (segment (start 125.856998 100.33) (end 125.475998 100.711) (width 0.2032) (layer B.Cu) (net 32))
 (segment (start 133.35 113.03) (end 125.475998 105.155998) (width 0.2032) (layer F.Cu) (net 32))
 (segment (start 125.475998 105.155998) (end 125.475998 101.276685) (width 0.2032) (layer F.Cu) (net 32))
 (segment (start 125.475998 101.276685) (end 125.475998 100.711) (width 0.2032) (layer F.Cu) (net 32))
 (via (at 126.4285 99.3775) (size 0.8) (drill 0.4) (layers F.Cu B.Cu) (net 33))
 (segment (start 130.42 99.06) (end 126.746 99.06) (width 0.2032) (layer B.Cu) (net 33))
 (segment (start 126.746 99.06) (end 126.4285 99.3775) (width 0.2032) (layer B.Cu) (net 33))
 (segment (start 126.4285 103.5685) (end 126.4285 99.943185) (width 0.2032) (layer F.Cu) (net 33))
 (segment (start 133.35 110.49) (end 126.4285 103.5685) (width 0.2032) (layer F.Cu) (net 33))
 (segment (start 126.4285 99.943185) (end 126.4285 99.3775) (width 0.2032) (layer F.Cu) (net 33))
 (via (at 127.3175 97.8535) (size 0.8) (drill 0.4) (layers F.Cu B.Cu) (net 34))
 (segment (start 130.42 97.79) (end 127.381 97.79) (width 0.2032) (layer B.Cu) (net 34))
 (segment (start 127.381 97.79) (end 127.3175 97.8535) (width 0.2032) (layer B.Cu) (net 34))
 (segment (start 127.323801 98.425486) (end 127.3175 98.419185) (width 0.2032) (layer F.Cu) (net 34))
 (segment (start 127.323801 101.923801) (end 127.323801 98.425486) (width 0.2032) (layer F.Cu) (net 34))
 (segment (start 133.35 107.95) (end 127.323801 101.923801) (width 0.2032) (layer F.Cu) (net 34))
 (segment (start 127.3175 98.419185) (end 127.3175 97.8535) (width 0.2032) (layer F.Cu) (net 34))
 (segment (start 131.699 125.73) (end 133.35 125.73) (width 0.2032) (layer B.Cu) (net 35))
 (segment (start 126.365 105.14) (end 126.365 120.396) (width 0.2032) (layer B.Cu) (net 35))
 (segment (start 126.365 120.396) (end 131.699 125.73) (width 0.2032) (layer B.Cu) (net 35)))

